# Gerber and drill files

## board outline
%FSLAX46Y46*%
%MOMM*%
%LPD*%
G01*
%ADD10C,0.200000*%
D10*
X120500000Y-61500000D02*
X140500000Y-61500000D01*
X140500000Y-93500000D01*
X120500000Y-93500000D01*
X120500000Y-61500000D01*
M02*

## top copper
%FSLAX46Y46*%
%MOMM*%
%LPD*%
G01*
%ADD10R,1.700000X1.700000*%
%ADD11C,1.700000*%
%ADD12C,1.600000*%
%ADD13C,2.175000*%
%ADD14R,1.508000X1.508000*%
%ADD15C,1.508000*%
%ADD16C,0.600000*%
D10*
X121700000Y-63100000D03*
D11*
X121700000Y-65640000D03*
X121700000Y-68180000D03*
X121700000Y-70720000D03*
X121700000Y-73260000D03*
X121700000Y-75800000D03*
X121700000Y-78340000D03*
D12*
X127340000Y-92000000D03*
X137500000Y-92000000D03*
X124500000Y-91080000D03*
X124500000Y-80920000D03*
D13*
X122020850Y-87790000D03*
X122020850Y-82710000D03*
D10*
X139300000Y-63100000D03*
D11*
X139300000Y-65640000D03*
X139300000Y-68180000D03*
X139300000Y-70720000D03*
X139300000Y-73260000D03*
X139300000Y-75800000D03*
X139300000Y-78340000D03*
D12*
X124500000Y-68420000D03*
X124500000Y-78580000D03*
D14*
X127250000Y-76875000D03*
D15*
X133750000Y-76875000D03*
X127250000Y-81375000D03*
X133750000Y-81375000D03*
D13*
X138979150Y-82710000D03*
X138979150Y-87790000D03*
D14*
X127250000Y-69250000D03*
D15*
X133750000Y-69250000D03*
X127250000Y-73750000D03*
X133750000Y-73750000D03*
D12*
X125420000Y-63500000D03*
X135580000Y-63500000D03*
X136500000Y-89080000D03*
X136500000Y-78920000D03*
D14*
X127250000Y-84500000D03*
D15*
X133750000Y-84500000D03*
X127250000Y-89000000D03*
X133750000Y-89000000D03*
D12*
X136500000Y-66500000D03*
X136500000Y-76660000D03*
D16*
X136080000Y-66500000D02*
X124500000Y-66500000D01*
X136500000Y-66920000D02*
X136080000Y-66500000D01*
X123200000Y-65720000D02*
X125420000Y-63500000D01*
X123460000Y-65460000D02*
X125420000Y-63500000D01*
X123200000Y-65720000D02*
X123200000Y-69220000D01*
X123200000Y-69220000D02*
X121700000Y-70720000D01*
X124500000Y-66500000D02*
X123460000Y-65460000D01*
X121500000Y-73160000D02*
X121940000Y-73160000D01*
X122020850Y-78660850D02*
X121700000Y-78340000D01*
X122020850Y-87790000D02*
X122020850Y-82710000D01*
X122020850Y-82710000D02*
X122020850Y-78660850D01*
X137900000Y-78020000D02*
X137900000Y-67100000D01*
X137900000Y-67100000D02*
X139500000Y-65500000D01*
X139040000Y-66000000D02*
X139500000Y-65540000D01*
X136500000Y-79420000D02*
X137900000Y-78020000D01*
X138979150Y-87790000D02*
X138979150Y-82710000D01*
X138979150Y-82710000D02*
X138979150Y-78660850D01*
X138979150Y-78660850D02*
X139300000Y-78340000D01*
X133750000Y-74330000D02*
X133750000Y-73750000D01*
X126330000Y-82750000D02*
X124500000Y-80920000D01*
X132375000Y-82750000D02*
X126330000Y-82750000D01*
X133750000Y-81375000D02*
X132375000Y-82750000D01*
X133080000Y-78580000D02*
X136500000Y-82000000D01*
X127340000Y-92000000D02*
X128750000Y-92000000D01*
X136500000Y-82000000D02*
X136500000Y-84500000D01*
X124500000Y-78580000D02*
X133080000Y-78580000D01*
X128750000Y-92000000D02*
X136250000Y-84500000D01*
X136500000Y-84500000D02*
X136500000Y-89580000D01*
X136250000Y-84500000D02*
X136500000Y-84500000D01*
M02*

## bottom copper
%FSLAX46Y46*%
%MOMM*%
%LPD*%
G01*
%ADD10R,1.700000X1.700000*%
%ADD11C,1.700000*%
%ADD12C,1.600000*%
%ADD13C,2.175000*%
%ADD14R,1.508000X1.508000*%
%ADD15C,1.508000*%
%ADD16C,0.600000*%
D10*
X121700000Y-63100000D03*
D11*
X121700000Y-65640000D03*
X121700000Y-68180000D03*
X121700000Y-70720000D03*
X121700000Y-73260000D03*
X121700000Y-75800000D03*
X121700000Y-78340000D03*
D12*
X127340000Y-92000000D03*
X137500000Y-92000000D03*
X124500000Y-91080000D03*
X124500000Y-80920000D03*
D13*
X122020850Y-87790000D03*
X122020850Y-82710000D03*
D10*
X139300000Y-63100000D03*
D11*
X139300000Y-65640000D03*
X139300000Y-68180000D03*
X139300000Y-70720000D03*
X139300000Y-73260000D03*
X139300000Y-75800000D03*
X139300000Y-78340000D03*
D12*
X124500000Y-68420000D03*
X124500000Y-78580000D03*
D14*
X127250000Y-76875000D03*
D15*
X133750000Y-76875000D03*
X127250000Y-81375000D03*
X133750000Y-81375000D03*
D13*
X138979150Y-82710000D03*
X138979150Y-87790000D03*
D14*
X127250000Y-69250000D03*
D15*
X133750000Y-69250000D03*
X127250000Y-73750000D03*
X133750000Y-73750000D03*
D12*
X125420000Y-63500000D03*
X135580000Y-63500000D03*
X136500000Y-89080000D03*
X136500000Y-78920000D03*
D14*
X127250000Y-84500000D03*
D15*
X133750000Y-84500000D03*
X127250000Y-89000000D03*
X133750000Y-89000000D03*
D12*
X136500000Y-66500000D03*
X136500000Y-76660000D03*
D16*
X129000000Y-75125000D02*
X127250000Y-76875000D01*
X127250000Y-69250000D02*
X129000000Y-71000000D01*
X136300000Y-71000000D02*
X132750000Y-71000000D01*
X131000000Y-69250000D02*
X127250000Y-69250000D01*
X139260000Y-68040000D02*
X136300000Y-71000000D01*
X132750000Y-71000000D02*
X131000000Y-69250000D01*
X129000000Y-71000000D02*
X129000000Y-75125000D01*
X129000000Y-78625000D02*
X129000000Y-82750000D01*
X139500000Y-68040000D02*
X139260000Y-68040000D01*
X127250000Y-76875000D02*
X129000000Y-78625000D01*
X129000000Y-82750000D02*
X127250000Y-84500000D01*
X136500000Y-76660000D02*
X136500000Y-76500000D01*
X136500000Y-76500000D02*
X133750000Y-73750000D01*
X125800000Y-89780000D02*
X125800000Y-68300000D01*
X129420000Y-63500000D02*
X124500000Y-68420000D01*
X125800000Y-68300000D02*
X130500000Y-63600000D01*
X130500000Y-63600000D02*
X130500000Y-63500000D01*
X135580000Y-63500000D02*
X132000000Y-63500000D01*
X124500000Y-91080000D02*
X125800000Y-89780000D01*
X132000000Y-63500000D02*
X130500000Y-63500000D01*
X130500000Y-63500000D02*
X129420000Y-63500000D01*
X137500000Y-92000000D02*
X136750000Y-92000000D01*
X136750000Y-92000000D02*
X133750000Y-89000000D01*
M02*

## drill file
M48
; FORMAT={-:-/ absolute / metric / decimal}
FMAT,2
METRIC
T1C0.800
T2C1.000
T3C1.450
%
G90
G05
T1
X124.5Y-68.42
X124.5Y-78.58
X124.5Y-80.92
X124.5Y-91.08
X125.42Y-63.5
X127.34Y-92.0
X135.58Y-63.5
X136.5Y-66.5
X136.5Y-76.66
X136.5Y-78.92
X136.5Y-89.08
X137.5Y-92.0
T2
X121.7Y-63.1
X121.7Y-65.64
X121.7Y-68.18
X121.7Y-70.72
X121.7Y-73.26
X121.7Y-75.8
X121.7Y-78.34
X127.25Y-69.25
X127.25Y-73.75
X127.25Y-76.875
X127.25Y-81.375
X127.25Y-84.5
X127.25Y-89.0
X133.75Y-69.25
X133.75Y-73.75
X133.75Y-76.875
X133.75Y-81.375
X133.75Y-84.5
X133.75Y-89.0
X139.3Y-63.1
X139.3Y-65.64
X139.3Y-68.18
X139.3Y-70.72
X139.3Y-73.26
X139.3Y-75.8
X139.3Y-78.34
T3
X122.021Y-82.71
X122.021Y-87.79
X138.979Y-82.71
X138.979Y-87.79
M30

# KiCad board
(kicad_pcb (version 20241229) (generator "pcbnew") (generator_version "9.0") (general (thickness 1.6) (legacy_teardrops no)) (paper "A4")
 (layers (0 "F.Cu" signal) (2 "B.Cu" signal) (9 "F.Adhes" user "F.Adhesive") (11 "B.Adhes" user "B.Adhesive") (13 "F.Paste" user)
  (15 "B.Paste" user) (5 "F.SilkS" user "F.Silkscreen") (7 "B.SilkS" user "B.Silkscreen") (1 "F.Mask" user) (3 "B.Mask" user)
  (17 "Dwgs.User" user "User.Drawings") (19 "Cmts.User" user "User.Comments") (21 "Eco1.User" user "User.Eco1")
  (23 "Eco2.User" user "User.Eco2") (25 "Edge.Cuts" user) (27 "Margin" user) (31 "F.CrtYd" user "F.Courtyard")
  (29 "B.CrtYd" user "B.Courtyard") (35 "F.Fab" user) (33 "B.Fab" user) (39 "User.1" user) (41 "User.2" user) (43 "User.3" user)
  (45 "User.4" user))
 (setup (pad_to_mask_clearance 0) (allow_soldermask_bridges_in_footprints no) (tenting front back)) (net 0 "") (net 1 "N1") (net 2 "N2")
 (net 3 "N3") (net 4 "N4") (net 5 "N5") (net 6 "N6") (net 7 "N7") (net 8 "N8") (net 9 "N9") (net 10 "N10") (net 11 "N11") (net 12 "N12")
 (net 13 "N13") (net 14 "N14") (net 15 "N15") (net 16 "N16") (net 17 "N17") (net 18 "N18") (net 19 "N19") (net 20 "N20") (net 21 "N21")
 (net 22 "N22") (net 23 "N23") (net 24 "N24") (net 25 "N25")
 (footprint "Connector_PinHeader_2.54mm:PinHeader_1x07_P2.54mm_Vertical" (layer "F.Cu") (at 121.7 63.1)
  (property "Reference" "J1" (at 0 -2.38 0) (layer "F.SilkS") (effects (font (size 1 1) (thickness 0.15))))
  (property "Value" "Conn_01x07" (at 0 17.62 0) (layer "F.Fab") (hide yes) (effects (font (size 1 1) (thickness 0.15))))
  (pad "1" thru_hole rect (at 0 0) (size 1.7 1.7) (drill 1) (layers "*.Cu" "*.Mask") (remove_unused_layers no) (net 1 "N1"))
  (pad "2" thru_hole circle (at 0 2.54) (size 1.7 1.7) (drill 1) (layers "*.Cu" "*.Mask") (remove_unused_layers no) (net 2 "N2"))
  (pad "3" thru_hole circle (at 0 5.08) (size 1.7 1.7) (drill 1) (layers "*.Cu" "*.Mask") (remove_unused_layers no) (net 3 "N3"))
  (pad "4" thru_hole circle (at 0 7.62) (size 1.7 1.7) (drill 1) (layers "*.Cu" "*.Mask") (remove_unused_layers no) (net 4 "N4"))
  (pad "5" thru_hole circle (at 0 10.16) (size 1.7 1.7) (drill 1) (layers "*.Cu" "*.Mask") (remove_unused_layers no) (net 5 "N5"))
  (pad "6" thru_hole circle (at 0 12.7) (size 1.7 1.7) (drill 1) (layers "*.Cu" "*.Mask") (remove_unused_layers no) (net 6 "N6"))
  (pad "7" thru_hole circle (at 0 15.24) (size 1.7 1.7) (drill 1) (layers "*.Cu" "*.Mask") (remove_unused_layers no) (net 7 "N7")))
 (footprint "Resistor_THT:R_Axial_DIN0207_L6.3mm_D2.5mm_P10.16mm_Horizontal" (layer "F.Cu") (at 127.34 92)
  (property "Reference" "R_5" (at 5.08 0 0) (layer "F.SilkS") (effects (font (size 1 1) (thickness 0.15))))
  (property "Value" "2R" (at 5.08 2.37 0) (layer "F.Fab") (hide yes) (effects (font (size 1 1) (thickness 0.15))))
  (pad "1" thru_hole circle (at 0 0) (size 1.6 1.6) (drill 0.8) (layers "*.Cu" "*.Mask") (remove_unused_layers no) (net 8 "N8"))
  (pad "2" thru_hole circle (at 10.16 0) (size 1.6 1.6) (drill 0.8) (layers "*.Cu" "*.Mask") (remove_unused_layers no) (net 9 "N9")))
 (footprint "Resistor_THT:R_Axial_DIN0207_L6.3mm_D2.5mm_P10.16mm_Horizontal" (layer "F.Cu") (at 124.5 91.08 90)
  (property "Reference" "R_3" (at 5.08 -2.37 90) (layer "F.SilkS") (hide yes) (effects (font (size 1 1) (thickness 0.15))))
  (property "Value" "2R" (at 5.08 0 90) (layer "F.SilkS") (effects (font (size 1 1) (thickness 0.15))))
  (pad "1" thru_hole circle (at 0 0 90) (size 1.6 1.6) (drill 0.8) (layers "*.Cu" "*.Mask") (remove_unused_layers no) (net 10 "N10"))
  (pad "2" thru_hole circle (at 10.16 0 90) (size 1.6 1.6) (drill 0.8) (layers "*.Cu" "*.Mask") (remove_unused_layers no) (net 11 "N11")))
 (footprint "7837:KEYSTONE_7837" (layer "F.Cu") (at 122.02085 85.25 90)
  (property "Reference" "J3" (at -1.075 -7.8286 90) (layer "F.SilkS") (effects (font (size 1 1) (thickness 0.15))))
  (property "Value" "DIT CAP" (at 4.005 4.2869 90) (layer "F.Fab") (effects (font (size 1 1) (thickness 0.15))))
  (pad "1_1" thru_hole circle (at -2.54 0 90) (size 2.175 2.175) (drill 1.45) (layers "*.Cu" "*.Mask") (remove_unused_layers no)
   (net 7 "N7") (solder_mask_margin 0.102))
  (pad "1_2" thru_hole circle (at 2.54 0 90) (size 2.175 2.175) (drill 1.45) (layers "*.Cu" "*.Mask") (remove_unused_layers no) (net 7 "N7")
   (solder_mask_margin 0.102)))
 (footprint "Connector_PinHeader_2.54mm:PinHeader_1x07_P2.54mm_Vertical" (layer "F.Cu") (at 139.3 63.1)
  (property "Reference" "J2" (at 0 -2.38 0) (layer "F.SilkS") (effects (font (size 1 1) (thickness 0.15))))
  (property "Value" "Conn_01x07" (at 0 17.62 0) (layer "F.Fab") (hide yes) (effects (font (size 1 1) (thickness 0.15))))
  (pad "1" thru_hole rect (at 0 0) (size 1.7 1.7) (drill 1) (layers "*.Cu" "*.Mask") (remove_unused_layers no) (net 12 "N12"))
  (pad "2" thru_hole circle (at 0 2.54) (size 1.7 1.7) (drill 1) (layers "*.Cu" "*.Mask") (remove_unused_layers no) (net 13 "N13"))
  (pad "3" thru_hole circle (at 0 5.08) (size 1.7 1.7) (drill 1) (layers "*.Cu" "*.Mask") (remove_unused_layers no) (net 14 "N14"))
  (pad "4" thru_hole circle (at 0 7.62) (size 1.7 1.7) (drill 1) (layers "*.Cu" "*.Mask") (remove_unused_layers no) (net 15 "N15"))
  (pad "5" thru_hole circle (at 0 10.16) (size 1.7 1.7) (drill 1) (layers "*.Cu" "*.Mask") (remove_unused_layers no) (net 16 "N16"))
  (pad "6" thru_hole circle (at 0 12.7) (size 1.7 1.7) (drill 1) (layers "*.Cu" "*.Mask") (remove_unused_layers no) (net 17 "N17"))
  (pad "7" thru_hole circle (at 0 15.24) (size 1.7 1.7) (drill 1) (layers "*.Cu" "*.Mask") (remove_unused_layers no) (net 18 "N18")))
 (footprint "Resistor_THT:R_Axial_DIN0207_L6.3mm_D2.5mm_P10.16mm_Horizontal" (layer "F.Cu") (at 124.5 68.42 -90)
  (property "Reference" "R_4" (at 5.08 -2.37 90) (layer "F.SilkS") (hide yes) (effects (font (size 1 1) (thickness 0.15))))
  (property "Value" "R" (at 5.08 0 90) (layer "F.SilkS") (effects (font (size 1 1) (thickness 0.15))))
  (pad "1" thru_hole circle (at 0 0 270) (size 1.6 1.6) (drill 0.8) (layers "*.Cu" "*.Mask") (remove_unused_layers no) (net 10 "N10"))
  (pad "2" thru_hole circle (at 10.16 0 270) (size 1.6 1.6) (drill 0.8) (layers "*.Cu" "*.Mask") (remove_unused_layers no) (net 8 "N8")))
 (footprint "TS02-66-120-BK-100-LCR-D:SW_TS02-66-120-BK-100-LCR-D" (layer "F.Cu") (at 130.5 79.125)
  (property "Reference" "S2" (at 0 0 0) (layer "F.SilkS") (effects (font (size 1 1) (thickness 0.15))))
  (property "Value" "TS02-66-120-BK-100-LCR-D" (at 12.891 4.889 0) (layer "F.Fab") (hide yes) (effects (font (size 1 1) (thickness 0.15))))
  (pad "1" thru_hole rect (at -3.25 -2.25) (size 1.508 1.508) (drill 1) (layers "*.Cu" "*.Mask") (remove_unused_layers no) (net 14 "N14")
   (solder_mask_margin 0.102))
  (pad "2" thru_hole circle (at 3.25 -2.25) (size 1.508 1.508) (drill 1) (layers "*.Cu" "*.Mask") (remove_unused_layers no) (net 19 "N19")
   (solder_mask_margin 0.102))
  (pad "3" thru_hole circle (at -3.25 2.25) (size 1.508 1.508) (drill 1) (layers "*.Cu" "*.Mask") (remove_unused_layers no) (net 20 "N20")
   (solder_mask_margin 0.102))
  (pad "4" thru_hole circle (at 3.25 2.25) (size 1.508 1.508) (drill 1) (layers "*.Cu" "*.Mask") (remove_unused_layers no) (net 11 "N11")
   (solder_mask_margin 0.102)))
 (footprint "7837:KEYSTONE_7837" (layer "F.Cu") (at 138.97915 85.25 -90)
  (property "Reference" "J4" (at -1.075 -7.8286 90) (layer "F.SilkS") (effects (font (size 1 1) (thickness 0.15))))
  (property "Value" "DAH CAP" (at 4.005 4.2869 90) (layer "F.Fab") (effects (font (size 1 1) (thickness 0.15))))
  (pad "1_1" thru_hole circle (at -2.54 0 270) (size 2.175 2.175) (drill 1.45) (layers "*.Cu" "*.Mask") (remove_unused_layers no)
   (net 18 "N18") (solder_mask_margin 0.102))
  (pad "1_2" thru_hole circle (at 2.54 0 270) (size 2.175 2.175) (drill 1.45) (layers "*.Cu" "*.Mask") (remove_unused_layers no)
   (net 18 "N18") (solder_mask_margin 0.102)))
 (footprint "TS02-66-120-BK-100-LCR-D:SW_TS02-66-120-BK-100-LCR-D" (layer "F.Cu") (at 130.5 71.5)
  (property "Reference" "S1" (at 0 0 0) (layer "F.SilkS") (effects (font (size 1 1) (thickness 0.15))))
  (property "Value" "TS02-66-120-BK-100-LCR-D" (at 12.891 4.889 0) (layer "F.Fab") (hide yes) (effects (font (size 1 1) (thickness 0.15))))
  (pad "1" thru_hole rect (at -3.25 -2.25) (size 1.508 1.508) (drill 1) (layers "*.Cu" "*.Mask") (remove_unused_layers no) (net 14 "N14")
   (solder_mask_margin 0.102))
  (pad "2" thru_hole circle (at 3.25 -2.25) (size 1.508 1.508) (drill 1) (layers "*.Cu" "*.Mask") (remove_unused_layers no) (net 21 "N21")
   (solder_mask_margin 0.102))
  (pad "3" thru_hole circle (at -3.25 2.25) (size 1.508 1.508) (drill 1) (layers "*.Cu" "*.Mask") (remove_unused_layers no) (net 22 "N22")
   (solder_mask_margin 0.102))
  (pad "4" thru_hole circle (at 3.25 2.25) (size 1.508 1.508) (drill 1) (layers "*.Cu" "*.Mask") (remove_unused_layers no) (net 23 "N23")
   (solder_mask_margin 0.102)))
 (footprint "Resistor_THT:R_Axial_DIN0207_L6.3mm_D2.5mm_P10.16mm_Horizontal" (layer "F.Cu") (at 125.42 63.5)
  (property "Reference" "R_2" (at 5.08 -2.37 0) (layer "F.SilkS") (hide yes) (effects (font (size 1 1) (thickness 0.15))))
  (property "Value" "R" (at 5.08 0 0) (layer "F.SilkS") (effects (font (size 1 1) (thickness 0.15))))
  (pad "1" thru_hole circle (at 0 0) (size 1.6 1.6) (drill 0.8) (layers "*.Cu" "*.Mask") (remove_unused_layers no) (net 4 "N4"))
  (pad "2" thru_hole circle (at 10.16 0) (size 1.6 1.6) (drill 0.8) (layers "*.Cu" "*.Mask") (remove_unused_layers no) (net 10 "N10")))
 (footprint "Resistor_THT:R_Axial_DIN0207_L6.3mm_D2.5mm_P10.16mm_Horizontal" (layer "F.Cu") (at 136.5 89.08 90)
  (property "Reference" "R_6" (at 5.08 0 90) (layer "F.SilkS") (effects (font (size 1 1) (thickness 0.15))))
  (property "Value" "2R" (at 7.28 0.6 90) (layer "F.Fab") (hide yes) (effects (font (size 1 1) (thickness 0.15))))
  (pad "1" thru_hole circle (at 0 0 90) (size 1.6 1.6) (drill 0.8) (layers "*.Cu" "*.Mask") (remove_unused_layers no) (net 8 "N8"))
  (pad "2" thru_hole circle (at 10.16 0 90) (size 1.6 1.6) (drill 0.8) (layers "*.Cu" "*.Mask") (remove_unused_layers no) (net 13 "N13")))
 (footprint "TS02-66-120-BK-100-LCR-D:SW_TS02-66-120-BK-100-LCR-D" (layer "F.Cu") (at 130.5 86.75)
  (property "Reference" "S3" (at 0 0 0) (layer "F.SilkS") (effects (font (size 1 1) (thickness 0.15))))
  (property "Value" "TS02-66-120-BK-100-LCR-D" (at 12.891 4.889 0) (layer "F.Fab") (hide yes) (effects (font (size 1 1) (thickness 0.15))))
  (pad "1" thru_hole rect (at -3.25 -2.25) (size 1.508 1.508) (drill 1) (layers "*.Cu" "*.Mask") (remove_unused_layers no) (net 14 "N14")
   (solder_mask_margin 0.102))
  (pad "2" thru_hole circle (at 3.25 -2.25) (size 1.508 1.508) (drill 1) (layers "*.Cu" "*.Mask") (remove_unused_layers no) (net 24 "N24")
   (solder_mask_margin 0.102))
  (pad "3" thru_hole circle (at -3.25 2.25) (size 1.508 1.508) (drill 1) (layers "*.Cu" "*.Mask") (remove_unused_layers no) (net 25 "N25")
   (solder_mask_margin 0.102))
  (pad "4" thru_hole circle (at 3.25 2.25) (size 1.508 1.508) (drill 1) (layers "*.Cu" "*.Mask") (remove_unused_layers no) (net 9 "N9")
   (solder_mask_margin 0.102)))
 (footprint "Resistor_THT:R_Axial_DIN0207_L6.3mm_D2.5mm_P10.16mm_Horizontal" (layer "F.Cu") (at 136.5 66.5 -90)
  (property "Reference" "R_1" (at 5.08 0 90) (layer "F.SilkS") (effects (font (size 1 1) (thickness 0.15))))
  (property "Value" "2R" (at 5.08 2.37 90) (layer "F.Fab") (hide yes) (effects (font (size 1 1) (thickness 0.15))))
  (pad "1" thru_hole circle (at 0 0 270) (size 1.6 1.6) (drill 0.8) (layers "*.Cu" "*.Mask") (remove_unused_layers no) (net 4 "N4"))
  (pad "2" thru_hole circle (at 10.16 0 270) (size 1.6 1.6) (drill 0.8) (layers "*.Cu" "*.Mask") (remove_unused_layers no) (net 23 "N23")))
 (gr_rect (start 120.5 61.5) (end 140.5 93.5) (stroke (width 0.2) (type solid)) (fill no) (layer "Edge.Cuts"))
 (segment (start 136.08 66.5) (end 124.5 66.5) (width 0.6) (layer "F.Cu") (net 4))
 (segment (start 136.5 66.92) (end 136.08 66.5) (width 0.6) (layer "F.Cu") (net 4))
 (segment (start 123.2 65.72) (end 125.42 63.5) (width 0.6) (layer "F.Cu") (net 4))
 (segment (start 123.46 65.46) (end 125.42 63.5) (width 0.6) (layer "F.Cu") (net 4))
 (segment (start 123.2 65.72) (end 123.2 69.22) (width 0.6) (layer "F.Cu") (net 4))
 (segment (start 123.2 69.22) (end 121.7 70.72) (width 0.6) (layer "F.Cu") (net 4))
 (segment (start 124.5 66.5) (end 123.46 65.46) (width 0.6) (layer "F.Cu") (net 4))
 (segment (start 121.5 73.16) (end 121.94 73.16) (width 0.6) (layer "F.Cu") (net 5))
 (segment (start 122.02085 78.66085) (end 121.7 78.34) (width 0.6) (layer "F.Cu") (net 7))
 (segment (start 122.02085 87.79) (end 122.02085 82.71) (width 0.6) (layer "F.Cu") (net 7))
 (segment (start 122.02085 82.71) (end 122.02085 78.66085) (width 0.6) (layer "F.Cu") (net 7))
 (segment (start 129 75.125) (end 127.25 76.875) (width 0.6) (layer "B.Cu") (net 14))
 (segment (start 127.25 69.25) (end 129 71) (width 0.6) (layer "B.Cu") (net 14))
 (segment (start 136.3 71) (end 132.75 71) (width 0.6) (layer "B.Cu") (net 14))
 (segment (start 131 69.25) (end 127.25 69.25) (width 0.6) (layer "B.Cu") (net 14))
 (segment (start 139.26 68.04) (end 136.3 71) (width 0.6) (layer "B.Cu") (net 14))
 (segment (start 132.75 71) (end 131 69.25) (width 0.6) (layer "B.Cu") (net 14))
 (segment (start 129 71) (end 129 75.125) (width 0.6) (layer "B.Cu") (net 14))
 (segment (start 129 78.625) (end 129 82.75) (width 0.6) (layer "B.Cu") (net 14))
 (segment (start 139.5 68.04) (end 139.26 68.04) (width 0.6) (layer "B.Cu") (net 14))
 (segment (start 127.25 76.875) (end 129 78.625) (width 0.6) (layer "B.Cu") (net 14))
 (segment (start 129 82.75) (end 127.25 84.5) (width 0.6) (layer "B.Cu") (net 14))
 (segment (start 137.9 78.02) (end 137.9 67.1) (width 0.6) (layer "F.Cu") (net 13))
 (segment (start 137.9 67.1) (end 139.5 65.5) (width 0.6) (layer "F.Cu") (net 13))
 (segment (start 139.04 66) (end 139.5 65.54) (width 0.6) (layer "F.Cu") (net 13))
 (segment (start 136.5 79.42) (end 137.9 78.02) (width 0.6) (layer "F.Cu") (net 13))
 (segment (start 138.97915 87.79) (end 138.97915 82.71) (width 0.6) (layer "F.Cu") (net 18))
 (segment (start 138.97915 82.71) (end 138.97915 78.66085) (width 0.6) (layer "F.Cu") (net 18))
 (segment (start 138.97915 78.66085) (end 139.3 78.34) (width 0.6) (layer "F.Cu") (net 18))
 (segment (start 133.75 74.33) (end 133.75 73.75) (width 0.6) (layer "F.Cu") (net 23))
 (segment (start 136.5 76.66) (end 136.5 76.5) (width 0.6) (layer "B.Cu") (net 23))
 (segment (start 136.5 76.5) (end 133.75 73.75) (width 0.6) (layer "B.Cu") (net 23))
 (segment (start 125.8 89.78) (end 125.8 68.3) (width 0.6) (layer "B.Cu") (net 10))
 (segment (start 129.42 63.5) (end 124.5 68.42) (width 0.6) (layer "B.Cu") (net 10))
 (segment (start 125.8 68.3) (end 130.5 63.6) (width 0.6) (layer "B.Cu") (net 10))
 (segment (start 130.5 63.6) (end 130.5 63.5) (width 0.6) (layer "B.Cu") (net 10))
 (segment (start 135.58 63.5) (end 132 63.5) (width 0.6) (layer "B.Cu") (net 10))
 (segment (start 124.5 91.08) (end 125.8 89.78) (width 0.6) (layer "B.Cu") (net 10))
 (segment (start 132 63.5) (end 130.5 63.5) (width 0.6) (layer "B.Cu") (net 10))
 (segment (start 130.5 63.5) (end 129.42 63.5) (width 0.6) (layer "B.Cu") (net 10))
 (segment (start 126.33 82.75) (end 124.5 80.92) (width 0.6) (layer "F.Cu") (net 11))
 (segment (start 132.375 82.75) (end 126.33 82.75) (width 0.6) (layer "F.Cu") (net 11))
 (segment (start 133.75 81.375) (end 132.375 82.75) (width 0.6) (layer "F.Cu") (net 11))
 (segment (start 133.08 78.58) (end 136.5 82) (width 0.6) (layer "F.Cu") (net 8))
 (segment (start 127.34 92) (end 128.75 92) (width 0.6) (layer "F.Cu") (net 8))
 (segment (start 136.5 82) (end 136.5 84.5) (width 0.6) (layer "F.Cu") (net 8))
 (segment (start 124.5 78.58) (end 133.08 78.58) (width 0.6) (layer "F.Cu") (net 8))
 (segment (start 128.75 92) (end 136.25 84.5) (width 0.6) (layer "F.Cu") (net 8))
 (segment (start 136.5 84.5) (end 136.5 89.58) (width 0.6) (layer "F.Cu") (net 8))
 (segment (start 136.25 84.5) (end 136.5 84.5) (width 0.6) (layer "F.Cu") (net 8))
 (segment (start 137.5 92) (end 136.75 92) (width 0.6) (layer "B.Cu") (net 9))
 (segment (start 136.75 92) (end 133.75 89) (width 0.6) (layer "B.Cu") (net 9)))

